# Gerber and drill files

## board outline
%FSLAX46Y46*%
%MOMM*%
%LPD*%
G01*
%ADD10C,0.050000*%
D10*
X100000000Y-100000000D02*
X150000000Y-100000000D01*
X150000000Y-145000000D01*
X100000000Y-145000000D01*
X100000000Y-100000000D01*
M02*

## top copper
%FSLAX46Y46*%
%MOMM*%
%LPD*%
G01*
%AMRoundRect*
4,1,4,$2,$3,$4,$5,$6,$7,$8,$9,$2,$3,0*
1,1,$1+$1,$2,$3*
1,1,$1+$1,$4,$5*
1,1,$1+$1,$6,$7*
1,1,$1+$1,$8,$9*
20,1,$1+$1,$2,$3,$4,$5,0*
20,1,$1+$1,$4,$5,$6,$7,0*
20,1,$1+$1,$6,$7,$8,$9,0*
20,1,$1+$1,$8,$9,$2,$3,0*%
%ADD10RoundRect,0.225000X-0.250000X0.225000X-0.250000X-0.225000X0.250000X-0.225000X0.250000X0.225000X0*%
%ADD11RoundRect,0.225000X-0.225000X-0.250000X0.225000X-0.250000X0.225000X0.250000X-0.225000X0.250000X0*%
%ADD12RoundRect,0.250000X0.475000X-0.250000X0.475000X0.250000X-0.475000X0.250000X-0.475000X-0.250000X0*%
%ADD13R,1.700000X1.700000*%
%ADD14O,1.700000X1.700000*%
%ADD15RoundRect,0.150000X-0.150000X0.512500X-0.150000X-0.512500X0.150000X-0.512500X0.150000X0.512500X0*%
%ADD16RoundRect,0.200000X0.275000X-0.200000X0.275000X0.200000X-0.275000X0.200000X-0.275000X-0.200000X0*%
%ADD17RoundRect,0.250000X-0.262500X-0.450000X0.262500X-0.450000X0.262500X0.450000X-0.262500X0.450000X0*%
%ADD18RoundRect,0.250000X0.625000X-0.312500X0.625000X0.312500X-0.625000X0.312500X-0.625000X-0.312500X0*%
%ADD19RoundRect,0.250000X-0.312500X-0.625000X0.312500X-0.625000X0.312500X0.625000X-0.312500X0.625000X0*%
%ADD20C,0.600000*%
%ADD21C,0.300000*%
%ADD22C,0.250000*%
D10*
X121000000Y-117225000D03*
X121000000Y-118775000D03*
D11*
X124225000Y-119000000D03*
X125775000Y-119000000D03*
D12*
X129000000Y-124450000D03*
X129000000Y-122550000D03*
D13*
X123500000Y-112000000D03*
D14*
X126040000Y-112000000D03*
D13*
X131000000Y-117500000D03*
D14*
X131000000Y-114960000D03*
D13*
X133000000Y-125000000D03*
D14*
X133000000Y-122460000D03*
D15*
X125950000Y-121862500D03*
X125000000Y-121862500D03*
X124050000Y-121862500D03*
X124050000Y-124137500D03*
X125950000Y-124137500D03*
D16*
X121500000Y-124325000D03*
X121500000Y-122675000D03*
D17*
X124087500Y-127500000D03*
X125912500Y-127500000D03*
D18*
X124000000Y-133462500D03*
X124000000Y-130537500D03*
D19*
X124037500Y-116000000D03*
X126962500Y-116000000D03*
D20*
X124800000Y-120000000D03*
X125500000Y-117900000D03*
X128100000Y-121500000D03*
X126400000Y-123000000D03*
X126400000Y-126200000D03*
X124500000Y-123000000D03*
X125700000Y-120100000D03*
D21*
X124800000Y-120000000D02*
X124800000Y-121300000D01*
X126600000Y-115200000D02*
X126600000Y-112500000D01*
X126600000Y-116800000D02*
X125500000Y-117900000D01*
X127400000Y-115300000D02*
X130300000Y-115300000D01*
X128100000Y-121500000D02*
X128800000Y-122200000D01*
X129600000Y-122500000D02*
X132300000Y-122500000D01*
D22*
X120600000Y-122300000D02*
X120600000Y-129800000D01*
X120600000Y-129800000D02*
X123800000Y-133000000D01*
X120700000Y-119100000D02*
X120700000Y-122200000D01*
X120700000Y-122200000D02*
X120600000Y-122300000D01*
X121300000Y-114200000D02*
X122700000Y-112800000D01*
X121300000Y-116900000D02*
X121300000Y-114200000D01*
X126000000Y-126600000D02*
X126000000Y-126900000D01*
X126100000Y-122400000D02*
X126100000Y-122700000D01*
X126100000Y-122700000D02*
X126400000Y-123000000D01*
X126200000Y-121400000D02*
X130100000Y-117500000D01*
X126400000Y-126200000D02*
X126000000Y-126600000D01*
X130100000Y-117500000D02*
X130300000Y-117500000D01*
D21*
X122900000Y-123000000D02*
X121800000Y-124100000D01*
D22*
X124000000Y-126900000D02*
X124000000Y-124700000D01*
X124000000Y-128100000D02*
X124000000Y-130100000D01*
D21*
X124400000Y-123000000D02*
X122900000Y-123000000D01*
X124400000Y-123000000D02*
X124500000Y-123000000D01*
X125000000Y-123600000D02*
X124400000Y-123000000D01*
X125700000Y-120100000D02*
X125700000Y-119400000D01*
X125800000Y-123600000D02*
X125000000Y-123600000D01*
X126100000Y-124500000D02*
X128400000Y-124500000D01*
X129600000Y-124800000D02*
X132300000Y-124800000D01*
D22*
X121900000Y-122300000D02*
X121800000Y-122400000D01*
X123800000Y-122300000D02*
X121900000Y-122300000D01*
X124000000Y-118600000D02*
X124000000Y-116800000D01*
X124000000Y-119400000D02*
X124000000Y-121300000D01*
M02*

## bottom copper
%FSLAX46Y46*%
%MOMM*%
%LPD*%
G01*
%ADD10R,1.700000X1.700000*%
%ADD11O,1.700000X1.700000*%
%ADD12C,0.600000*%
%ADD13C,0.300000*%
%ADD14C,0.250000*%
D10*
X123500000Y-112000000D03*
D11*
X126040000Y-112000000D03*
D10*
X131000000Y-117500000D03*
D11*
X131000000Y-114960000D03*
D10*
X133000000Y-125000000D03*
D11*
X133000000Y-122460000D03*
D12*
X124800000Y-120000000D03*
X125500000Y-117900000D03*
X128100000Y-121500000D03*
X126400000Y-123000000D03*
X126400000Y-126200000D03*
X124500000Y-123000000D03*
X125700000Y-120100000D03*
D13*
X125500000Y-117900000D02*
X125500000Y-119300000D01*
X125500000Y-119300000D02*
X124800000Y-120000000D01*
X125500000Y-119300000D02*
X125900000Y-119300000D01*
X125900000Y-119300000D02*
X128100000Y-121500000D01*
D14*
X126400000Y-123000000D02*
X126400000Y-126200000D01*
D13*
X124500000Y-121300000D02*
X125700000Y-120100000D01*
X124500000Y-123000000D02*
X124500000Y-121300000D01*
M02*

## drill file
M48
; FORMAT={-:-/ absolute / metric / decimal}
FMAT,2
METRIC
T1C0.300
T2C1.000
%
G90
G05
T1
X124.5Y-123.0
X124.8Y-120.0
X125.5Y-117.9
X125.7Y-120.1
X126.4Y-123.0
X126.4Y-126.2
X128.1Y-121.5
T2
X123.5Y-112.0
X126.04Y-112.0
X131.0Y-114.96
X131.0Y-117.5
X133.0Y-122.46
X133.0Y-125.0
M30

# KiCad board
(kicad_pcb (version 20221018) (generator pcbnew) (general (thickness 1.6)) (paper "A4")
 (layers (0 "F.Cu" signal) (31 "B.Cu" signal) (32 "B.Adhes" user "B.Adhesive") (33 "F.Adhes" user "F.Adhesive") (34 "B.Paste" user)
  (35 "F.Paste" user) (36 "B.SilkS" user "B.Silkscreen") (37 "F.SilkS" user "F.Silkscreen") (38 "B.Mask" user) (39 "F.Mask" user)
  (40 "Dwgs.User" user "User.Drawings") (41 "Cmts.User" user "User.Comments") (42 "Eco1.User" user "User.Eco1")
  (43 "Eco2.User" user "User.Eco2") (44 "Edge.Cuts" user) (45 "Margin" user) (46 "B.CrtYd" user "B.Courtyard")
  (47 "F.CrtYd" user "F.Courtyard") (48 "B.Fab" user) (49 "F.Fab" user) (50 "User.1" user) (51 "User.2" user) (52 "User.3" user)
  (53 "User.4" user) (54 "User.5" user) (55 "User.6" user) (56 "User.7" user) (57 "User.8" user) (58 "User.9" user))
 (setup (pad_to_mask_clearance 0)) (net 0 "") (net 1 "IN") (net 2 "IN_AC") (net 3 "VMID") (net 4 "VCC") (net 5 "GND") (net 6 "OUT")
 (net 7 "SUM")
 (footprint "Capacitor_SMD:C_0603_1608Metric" (layer "F.Cu") (at 121 118 -90)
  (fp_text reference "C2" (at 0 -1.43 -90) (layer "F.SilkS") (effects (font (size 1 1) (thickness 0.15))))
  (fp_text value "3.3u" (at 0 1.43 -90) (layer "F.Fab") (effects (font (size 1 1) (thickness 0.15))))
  (pad "1" smd roundrect (at -0.775 0 270) (size 0.9 0.95) (layers "F.Cu" "F.Paste" "F.Mask") (roundrect_rratio 0.25) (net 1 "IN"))
  (pad "2" smd roundrect (at 0.775 0 270) (size 0.9 0.95) (layers "F.Cu" "F.Paste" "F.Mask") (roundrect_rratio 0.25) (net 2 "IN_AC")))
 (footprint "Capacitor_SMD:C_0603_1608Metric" (layer "F.Cu") (at 125 119)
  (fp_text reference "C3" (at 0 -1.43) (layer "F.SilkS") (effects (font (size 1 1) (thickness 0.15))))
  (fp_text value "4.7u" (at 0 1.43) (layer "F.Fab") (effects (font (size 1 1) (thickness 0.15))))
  (pad "1" smd roundrect (at -0.775 0) (size 0.9 0.95) (layers "F.Cu" "F.Paste" "F.Mask") (roundrect_rratio 0.25) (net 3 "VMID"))
  (pad "2" smd roundrect (at 0.775 0) (size 0.9 0.95) (layers "F.Cu" "F.Paste" "F.Mask") (roundrect_rratio 0.25) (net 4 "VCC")))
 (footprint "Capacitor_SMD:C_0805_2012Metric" (layer "F.Cu") (at 129 123.5 90)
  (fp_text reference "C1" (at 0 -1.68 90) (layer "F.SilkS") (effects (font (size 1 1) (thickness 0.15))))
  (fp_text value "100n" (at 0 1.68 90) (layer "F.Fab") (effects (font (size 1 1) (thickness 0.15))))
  (pad "1" smd roundrect (at -0.95 0 90) (size 1 1.45) (layers "F.Cu" "F.Paste" "F.Mask") (roundrect_rratio 0.25) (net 4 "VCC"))
  (pad "2" smd roundrect (at 0.95 0 90) (size 1 1.45) (layers "F.Cu" "F.Paste" "F.Mask") (roundrect_rratio 0.25) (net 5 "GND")))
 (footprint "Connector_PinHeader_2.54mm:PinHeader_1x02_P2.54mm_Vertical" (layer "F.Cu") (at 123.5 112 90)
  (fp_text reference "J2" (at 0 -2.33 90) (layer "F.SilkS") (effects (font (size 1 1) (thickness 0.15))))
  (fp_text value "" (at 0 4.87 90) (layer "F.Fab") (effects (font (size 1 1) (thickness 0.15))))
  (pad "1" thru_hole rect (at 0 0 90) (size 1.7 1.7) (drill 1) (layers "*.Cu" "*.Mask") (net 1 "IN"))
  (pad "2" thru_hole oval (at 0 2.54 90) (size 1.7 1.7) (drill 1) (layers "*.Cu" "*.Mask") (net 5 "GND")))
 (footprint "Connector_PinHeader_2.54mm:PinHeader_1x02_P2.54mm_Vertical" (layer "F.Cu") (at 131 117.5 180)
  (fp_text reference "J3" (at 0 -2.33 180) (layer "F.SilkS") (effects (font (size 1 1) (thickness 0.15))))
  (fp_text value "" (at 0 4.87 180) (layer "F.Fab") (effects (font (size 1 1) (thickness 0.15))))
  (pad "1" thru_hole rect (at 0 0 180) (size 1.7 1.7) (drill 1) (layers "*.Cu" "*.Mask") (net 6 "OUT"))
  (pad "2" thru_hole oval (at 0 2.54 180) (size 1.7 1.7) (drill 1) (layers "*.Cu" "*.Mask") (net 5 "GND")))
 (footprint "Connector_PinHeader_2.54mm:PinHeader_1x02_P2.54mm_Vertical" (layer "F.Cu") (at 133 125 180)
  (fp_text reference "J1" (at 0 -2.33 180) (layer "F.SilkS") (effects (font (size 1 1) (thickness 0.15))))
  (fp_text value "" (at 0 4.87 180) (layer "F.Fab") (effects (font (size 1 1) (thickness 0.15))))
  (pad "1" thru_hole rect (at 0 0 180) (size 1.7 1.7) (drill 1) (layers "*.Cu" "*.Mask") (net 4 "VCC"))
  (pad "2" thru_hole oval (at 0 2.54 180) (size 1.7 1.7) (drill 1) (layers "*.Cu" "*.Mask") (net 5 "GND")))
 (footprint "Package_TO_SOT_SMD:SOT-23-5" (layer "F.Cu") (at 125 123 -90)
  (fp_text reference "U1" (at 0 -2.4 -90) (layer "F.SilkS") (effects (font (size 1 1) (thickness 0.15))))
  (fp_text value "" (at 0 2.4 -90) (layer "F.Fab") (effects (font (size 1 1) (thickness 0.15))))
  (pad "1" smd roundrect (at -1.1375 -0.95 270) (size 1.325 0.6) (layers "F.Cu" "F.Paste" "F.Mask") (roundrect_rratio 0.25) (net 6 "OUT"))
  (pad "2" smd roundrect (at -1.1375 0 270) (size 1.325 0.6) (layers "F.Cu" "F.Paste" "F.Mask") (roundrect_rratio 0.25) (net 5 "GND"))
  (pad "3" smd roundrect (at -1.1375 0.95 270) (size 1.325 0.6) (layers "F.Cu" "F.Paste" "F.Mask") (roundrect_rratio 0.25) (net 3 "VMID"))
  (pad "4" smd roundrect (at 1.1375 0.95 270) (size 1.325 0.6) (layers "F.Cu" "F.Paste" "F.Mask") (roundrect_rratio 0.25) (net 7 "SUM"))
  (pad "5" smd roundrect (at 1.1375 -0.95 270) (size 1.325 0.6) (layers "F.Cu" "F.Paste" "F.Mask") (roundrect_rratio 0.25) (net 4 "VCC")))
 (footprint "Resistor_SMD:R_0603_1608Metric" (layer "F.Cu") (at 121.5 123.5 90)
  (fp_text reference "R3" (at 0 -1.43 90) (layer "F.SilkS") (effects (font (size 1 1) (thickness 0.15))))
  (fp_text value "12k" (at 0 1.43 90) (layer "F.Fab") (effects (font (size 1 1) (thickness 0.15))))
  (pad "1" smd roundrect (at -0.825 0 90) (size 0.8 0.95) (layers "F.Cu" "F.Paste" "F.Mask") (roundrect_rratio 0.25) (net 4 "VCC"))
  (pad "2" smd roundrect (at 0.825 0 90) (size 0.8 0.95) (layers "F.Cu" "F.Paste" "F.Mask") (roundrect_rratio 0.25) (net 3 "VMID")))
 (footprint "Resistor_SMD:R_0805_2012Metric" (layer "F.Cu") (at 125 127.5)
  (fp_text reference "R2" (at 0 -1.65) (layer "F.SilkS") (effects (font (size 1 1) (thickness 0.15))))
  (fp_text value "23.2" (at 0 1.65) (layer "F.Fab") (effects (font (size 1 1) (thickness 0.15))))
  (pad "1" smd roundrect (at -0.9125 0) (size 1.025 1.4) (layers "F.Cu" "F.Paste" "F.Mask") (roundrect_rratio 0.243902) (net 7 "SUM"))
  (pad "2" smd roundrect (at 0.9125 0) (size 1.025 1.4) (layers "F.Cu" "F.Paste" "F.Mask") (roundrect_rratio 0.243902) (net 6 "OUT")))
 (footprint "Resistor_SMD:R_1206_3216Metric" (layer "F.Cu") (at 124 132 90)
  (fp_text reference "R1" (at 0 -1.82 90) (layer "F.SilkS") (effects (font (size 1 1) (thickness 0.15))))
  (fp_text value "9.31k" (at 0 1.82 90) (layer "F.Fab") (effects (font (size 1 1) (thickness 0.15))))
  (pad "1" smd roundrect (at -1.4625 0 90) (size 1.125 1.75) (layers "F.Cu" "F.Paste" "F.Mask") (roundrect_rratio 0.222222) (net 2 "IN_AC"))
  (pad "2" smd roundrect (at 1.4625 0 90) (size 1.125 1.75) (layers "F.Cu" "F.Paste" "F.Mask") (roundrect_rratio 0.222222) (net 7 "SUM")))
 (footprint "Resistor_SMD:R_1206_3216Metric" (layer "F.Cu") (at 125.5 116)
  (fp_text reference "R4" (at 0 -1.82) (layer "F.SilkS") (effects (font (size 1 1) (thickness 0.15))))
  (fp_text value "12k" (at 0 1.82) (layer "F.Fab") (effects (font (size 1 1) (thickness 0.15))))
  (pad "1" smd roundrect (at -1.4625 0) (size 1.125 1.75) (layers "F.Cu" "F.Paste" "F.Mask") (roundrect_rratio 0.222222) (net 3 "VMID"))
  (pad "2" smd roundrect (at 1.4625 0) (size 1.125 1.75) (layers "F.Cu" "F.Paste" "F.Mask") (roundrect_rratio 0.222222) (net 5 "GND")))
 (gr_rect (start 100 100) (end 150 145) (stroke (width 0.05) (type default)) (fill none) (layer "Edge.Cuts"))
 (segment (start 124.8 120) (end 124.8 121.3) (width 0.3) (layer "F.Cu") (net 5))
 (segment (start 126.6 115.2) (end 126.6 112.5) (width 0.3) (layer "F.Cu") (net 5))
 (segment (start 126.6 116.8) (end 125.5 117.9) (width 0.3) (layer "F.Cu") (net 5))
 (segment (start 127.4 115.3) (end 130.3 115.3) (width 0.3) (layer "F.Cu") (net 5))
 (segment (start 128.1 121.5) (end 128.8 122.2) (width 0.3) (layer "F.Cu") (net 5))
 (segment (start 129.6 122.5) (end 132.3 122.5) (width 0.3) (layer "F.Cu") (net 5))
 (via (at 124.8 120) (size 0.6) (drill 0.3) (layers "F.Cu" "B.Cu") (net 5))
 (via (at 125.5 117.9) (size 0.6) (drill 0.3) (layers "F.Cu" "B.Cu") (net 5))
 (via (at 128.1 121.5) (size 0.6) (drill 0.3) (layers "F.Cu" "B.Cu") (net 5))
 (segment (start 120.6 122.3) (end 120.6 129.8) (width 0.25) (layer "F.Cu") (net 2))
 (segment (start 120.6 129.8) (end 123.8 133) (width 0.25) (layer "F.Cu") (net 2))
 (segment (start 120.7 119.1) (end 120.7 122.2) (width 0.25) (layer "F.Cu") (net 2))
 (segment (start 120.7 122.2) (end 120.6 122.3) (width 0.25) (layer "F.Cu") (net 2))
 (segment (start 121.3 114.2) (end 122.7 112.8) (width 0.25) (layer "F.Cu") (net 1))
 (segment (start 121.3 116.9) (end 121.3 114.2) (width 0.25) (layer "F.Cu") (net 1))
 (segment (start 125.5 117.9) (end 125.5 119.3) (width 0.3) (layer "B.Cu") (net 5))
 (segment (start 125.5 119.3) (end 124.8 120) (width 0.3) (layer "B.Cu") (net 5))
 (segment (start 125.5 119.3) (end 125.9 119.3) (width 0.3) (layer "B.Cu") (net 5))
 (segment (start 125.9 119.3) (end 128.1 121.5) (width 0.3) (layer "B.Cu") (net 5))
 (segment (start 126 126.6) (end 126 126.9) (width 0.25) (layer "F.Cu") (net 6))
 (segment (start 126.1 122.4) (end 126.1 122.7) (width 0.25) (layer "F.Cu") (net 6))
 (segment (start 126.1 122.7) (end 126.4 123) (width 0.25) (layer "F.Cu") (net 6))
 (segment (start 126.2 121.4) (end 130.1 117.5) (width 0.25) (layer "F.Cu") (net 6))
 (segment (start 126.4 126.2) (end 126 126.6) (width 0.25) (layer "F.Cu") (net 6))
 (segment (start 130.1 117.5) (end 130.3 117.5) (width 0.25) (layer "F.Cu") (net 6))
 (via (at 126.4 123) (size 0.6) (drill 0.3) (layers "F.Cu" "B.Cu") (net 6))
 (via (at 126.4 126.2) (size 0.6) (drill 0.3) (layers "F.Cu" "B.Cu") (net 6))
 (segment (start 122.9 123) (end 121.8 124.1) (width 0.3) (layer "F.Cu") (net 4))
 (segment (start 124 126.9) (end 124 124.7) (width 0.25) (layer "F.Cu") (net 7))
 (segment (start 124 128.1) (end 124 130.1) (width 0.25) (layer "F.Cu") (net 7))
 (segment (start 124.4 123) (end 122.9 123) (width 0.3) (layer "F.Cu") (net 4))
 (segment (start 124.4 123) (end 124.5 123) (width 0.3) (layer "F.Cu") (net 4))
 (segment (start 125 123.6) (end 124.4 123) (width 0.3) (layer "F.Cu") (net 4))
 (segment (start 125.7 120.1) (end 125.7 119.4) (width 0.3) (layer "F.Cu") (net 4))
 (segment (start 125.8 123.6) (end 125 123.6) (width 0.3) (layer "F.Cu") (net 4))
 (segment (start 126.1 124.5) (end 128.4 124.5) (width 0.3) (layer "F.Cu") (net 4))
 (segment (start 126.4 123) (end 126.4 126.2) (width 0.25) (layer "B.Cu") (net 6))
 (segment (start 129.6 124.8) (end 132.3 124.8) (width 0.3) (layer "F.Cu") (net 4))
 (via (at 124.5 123) (size 0.6) (drill 0.3) (layers "F.Cu" "B.Cu") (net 4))
 (via (at 125.7 120.1) (size 0.6) (drill 0.3) (layers "F.Cu" "B.Cu") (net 4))
 (segment (start 121.9 122.3) (end 121.8 122.4) (width 0.25) (layer "F.Cu") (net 3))
 (segment (start 123.8 122.3) (end 121.9 122.3) (width 0.25) (layer "F.Cu") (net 3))
 (segment (start 124 118.6) (end 124 116.8) (width 0.25) (layer "F.Cu") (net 3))
 (segment (start 124 119.4) (end 124 121.3) (width 0.25) (layer "F.Cu") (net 3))
 (segment (start 124.5 121.3) (end 125.7 120.1) (width 0.3) (layer "B.Cu") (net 4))
 (segment (start 124.5 123) (end 124.5 121.3) (width 0.3) (layer "B.Cu") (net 4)))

